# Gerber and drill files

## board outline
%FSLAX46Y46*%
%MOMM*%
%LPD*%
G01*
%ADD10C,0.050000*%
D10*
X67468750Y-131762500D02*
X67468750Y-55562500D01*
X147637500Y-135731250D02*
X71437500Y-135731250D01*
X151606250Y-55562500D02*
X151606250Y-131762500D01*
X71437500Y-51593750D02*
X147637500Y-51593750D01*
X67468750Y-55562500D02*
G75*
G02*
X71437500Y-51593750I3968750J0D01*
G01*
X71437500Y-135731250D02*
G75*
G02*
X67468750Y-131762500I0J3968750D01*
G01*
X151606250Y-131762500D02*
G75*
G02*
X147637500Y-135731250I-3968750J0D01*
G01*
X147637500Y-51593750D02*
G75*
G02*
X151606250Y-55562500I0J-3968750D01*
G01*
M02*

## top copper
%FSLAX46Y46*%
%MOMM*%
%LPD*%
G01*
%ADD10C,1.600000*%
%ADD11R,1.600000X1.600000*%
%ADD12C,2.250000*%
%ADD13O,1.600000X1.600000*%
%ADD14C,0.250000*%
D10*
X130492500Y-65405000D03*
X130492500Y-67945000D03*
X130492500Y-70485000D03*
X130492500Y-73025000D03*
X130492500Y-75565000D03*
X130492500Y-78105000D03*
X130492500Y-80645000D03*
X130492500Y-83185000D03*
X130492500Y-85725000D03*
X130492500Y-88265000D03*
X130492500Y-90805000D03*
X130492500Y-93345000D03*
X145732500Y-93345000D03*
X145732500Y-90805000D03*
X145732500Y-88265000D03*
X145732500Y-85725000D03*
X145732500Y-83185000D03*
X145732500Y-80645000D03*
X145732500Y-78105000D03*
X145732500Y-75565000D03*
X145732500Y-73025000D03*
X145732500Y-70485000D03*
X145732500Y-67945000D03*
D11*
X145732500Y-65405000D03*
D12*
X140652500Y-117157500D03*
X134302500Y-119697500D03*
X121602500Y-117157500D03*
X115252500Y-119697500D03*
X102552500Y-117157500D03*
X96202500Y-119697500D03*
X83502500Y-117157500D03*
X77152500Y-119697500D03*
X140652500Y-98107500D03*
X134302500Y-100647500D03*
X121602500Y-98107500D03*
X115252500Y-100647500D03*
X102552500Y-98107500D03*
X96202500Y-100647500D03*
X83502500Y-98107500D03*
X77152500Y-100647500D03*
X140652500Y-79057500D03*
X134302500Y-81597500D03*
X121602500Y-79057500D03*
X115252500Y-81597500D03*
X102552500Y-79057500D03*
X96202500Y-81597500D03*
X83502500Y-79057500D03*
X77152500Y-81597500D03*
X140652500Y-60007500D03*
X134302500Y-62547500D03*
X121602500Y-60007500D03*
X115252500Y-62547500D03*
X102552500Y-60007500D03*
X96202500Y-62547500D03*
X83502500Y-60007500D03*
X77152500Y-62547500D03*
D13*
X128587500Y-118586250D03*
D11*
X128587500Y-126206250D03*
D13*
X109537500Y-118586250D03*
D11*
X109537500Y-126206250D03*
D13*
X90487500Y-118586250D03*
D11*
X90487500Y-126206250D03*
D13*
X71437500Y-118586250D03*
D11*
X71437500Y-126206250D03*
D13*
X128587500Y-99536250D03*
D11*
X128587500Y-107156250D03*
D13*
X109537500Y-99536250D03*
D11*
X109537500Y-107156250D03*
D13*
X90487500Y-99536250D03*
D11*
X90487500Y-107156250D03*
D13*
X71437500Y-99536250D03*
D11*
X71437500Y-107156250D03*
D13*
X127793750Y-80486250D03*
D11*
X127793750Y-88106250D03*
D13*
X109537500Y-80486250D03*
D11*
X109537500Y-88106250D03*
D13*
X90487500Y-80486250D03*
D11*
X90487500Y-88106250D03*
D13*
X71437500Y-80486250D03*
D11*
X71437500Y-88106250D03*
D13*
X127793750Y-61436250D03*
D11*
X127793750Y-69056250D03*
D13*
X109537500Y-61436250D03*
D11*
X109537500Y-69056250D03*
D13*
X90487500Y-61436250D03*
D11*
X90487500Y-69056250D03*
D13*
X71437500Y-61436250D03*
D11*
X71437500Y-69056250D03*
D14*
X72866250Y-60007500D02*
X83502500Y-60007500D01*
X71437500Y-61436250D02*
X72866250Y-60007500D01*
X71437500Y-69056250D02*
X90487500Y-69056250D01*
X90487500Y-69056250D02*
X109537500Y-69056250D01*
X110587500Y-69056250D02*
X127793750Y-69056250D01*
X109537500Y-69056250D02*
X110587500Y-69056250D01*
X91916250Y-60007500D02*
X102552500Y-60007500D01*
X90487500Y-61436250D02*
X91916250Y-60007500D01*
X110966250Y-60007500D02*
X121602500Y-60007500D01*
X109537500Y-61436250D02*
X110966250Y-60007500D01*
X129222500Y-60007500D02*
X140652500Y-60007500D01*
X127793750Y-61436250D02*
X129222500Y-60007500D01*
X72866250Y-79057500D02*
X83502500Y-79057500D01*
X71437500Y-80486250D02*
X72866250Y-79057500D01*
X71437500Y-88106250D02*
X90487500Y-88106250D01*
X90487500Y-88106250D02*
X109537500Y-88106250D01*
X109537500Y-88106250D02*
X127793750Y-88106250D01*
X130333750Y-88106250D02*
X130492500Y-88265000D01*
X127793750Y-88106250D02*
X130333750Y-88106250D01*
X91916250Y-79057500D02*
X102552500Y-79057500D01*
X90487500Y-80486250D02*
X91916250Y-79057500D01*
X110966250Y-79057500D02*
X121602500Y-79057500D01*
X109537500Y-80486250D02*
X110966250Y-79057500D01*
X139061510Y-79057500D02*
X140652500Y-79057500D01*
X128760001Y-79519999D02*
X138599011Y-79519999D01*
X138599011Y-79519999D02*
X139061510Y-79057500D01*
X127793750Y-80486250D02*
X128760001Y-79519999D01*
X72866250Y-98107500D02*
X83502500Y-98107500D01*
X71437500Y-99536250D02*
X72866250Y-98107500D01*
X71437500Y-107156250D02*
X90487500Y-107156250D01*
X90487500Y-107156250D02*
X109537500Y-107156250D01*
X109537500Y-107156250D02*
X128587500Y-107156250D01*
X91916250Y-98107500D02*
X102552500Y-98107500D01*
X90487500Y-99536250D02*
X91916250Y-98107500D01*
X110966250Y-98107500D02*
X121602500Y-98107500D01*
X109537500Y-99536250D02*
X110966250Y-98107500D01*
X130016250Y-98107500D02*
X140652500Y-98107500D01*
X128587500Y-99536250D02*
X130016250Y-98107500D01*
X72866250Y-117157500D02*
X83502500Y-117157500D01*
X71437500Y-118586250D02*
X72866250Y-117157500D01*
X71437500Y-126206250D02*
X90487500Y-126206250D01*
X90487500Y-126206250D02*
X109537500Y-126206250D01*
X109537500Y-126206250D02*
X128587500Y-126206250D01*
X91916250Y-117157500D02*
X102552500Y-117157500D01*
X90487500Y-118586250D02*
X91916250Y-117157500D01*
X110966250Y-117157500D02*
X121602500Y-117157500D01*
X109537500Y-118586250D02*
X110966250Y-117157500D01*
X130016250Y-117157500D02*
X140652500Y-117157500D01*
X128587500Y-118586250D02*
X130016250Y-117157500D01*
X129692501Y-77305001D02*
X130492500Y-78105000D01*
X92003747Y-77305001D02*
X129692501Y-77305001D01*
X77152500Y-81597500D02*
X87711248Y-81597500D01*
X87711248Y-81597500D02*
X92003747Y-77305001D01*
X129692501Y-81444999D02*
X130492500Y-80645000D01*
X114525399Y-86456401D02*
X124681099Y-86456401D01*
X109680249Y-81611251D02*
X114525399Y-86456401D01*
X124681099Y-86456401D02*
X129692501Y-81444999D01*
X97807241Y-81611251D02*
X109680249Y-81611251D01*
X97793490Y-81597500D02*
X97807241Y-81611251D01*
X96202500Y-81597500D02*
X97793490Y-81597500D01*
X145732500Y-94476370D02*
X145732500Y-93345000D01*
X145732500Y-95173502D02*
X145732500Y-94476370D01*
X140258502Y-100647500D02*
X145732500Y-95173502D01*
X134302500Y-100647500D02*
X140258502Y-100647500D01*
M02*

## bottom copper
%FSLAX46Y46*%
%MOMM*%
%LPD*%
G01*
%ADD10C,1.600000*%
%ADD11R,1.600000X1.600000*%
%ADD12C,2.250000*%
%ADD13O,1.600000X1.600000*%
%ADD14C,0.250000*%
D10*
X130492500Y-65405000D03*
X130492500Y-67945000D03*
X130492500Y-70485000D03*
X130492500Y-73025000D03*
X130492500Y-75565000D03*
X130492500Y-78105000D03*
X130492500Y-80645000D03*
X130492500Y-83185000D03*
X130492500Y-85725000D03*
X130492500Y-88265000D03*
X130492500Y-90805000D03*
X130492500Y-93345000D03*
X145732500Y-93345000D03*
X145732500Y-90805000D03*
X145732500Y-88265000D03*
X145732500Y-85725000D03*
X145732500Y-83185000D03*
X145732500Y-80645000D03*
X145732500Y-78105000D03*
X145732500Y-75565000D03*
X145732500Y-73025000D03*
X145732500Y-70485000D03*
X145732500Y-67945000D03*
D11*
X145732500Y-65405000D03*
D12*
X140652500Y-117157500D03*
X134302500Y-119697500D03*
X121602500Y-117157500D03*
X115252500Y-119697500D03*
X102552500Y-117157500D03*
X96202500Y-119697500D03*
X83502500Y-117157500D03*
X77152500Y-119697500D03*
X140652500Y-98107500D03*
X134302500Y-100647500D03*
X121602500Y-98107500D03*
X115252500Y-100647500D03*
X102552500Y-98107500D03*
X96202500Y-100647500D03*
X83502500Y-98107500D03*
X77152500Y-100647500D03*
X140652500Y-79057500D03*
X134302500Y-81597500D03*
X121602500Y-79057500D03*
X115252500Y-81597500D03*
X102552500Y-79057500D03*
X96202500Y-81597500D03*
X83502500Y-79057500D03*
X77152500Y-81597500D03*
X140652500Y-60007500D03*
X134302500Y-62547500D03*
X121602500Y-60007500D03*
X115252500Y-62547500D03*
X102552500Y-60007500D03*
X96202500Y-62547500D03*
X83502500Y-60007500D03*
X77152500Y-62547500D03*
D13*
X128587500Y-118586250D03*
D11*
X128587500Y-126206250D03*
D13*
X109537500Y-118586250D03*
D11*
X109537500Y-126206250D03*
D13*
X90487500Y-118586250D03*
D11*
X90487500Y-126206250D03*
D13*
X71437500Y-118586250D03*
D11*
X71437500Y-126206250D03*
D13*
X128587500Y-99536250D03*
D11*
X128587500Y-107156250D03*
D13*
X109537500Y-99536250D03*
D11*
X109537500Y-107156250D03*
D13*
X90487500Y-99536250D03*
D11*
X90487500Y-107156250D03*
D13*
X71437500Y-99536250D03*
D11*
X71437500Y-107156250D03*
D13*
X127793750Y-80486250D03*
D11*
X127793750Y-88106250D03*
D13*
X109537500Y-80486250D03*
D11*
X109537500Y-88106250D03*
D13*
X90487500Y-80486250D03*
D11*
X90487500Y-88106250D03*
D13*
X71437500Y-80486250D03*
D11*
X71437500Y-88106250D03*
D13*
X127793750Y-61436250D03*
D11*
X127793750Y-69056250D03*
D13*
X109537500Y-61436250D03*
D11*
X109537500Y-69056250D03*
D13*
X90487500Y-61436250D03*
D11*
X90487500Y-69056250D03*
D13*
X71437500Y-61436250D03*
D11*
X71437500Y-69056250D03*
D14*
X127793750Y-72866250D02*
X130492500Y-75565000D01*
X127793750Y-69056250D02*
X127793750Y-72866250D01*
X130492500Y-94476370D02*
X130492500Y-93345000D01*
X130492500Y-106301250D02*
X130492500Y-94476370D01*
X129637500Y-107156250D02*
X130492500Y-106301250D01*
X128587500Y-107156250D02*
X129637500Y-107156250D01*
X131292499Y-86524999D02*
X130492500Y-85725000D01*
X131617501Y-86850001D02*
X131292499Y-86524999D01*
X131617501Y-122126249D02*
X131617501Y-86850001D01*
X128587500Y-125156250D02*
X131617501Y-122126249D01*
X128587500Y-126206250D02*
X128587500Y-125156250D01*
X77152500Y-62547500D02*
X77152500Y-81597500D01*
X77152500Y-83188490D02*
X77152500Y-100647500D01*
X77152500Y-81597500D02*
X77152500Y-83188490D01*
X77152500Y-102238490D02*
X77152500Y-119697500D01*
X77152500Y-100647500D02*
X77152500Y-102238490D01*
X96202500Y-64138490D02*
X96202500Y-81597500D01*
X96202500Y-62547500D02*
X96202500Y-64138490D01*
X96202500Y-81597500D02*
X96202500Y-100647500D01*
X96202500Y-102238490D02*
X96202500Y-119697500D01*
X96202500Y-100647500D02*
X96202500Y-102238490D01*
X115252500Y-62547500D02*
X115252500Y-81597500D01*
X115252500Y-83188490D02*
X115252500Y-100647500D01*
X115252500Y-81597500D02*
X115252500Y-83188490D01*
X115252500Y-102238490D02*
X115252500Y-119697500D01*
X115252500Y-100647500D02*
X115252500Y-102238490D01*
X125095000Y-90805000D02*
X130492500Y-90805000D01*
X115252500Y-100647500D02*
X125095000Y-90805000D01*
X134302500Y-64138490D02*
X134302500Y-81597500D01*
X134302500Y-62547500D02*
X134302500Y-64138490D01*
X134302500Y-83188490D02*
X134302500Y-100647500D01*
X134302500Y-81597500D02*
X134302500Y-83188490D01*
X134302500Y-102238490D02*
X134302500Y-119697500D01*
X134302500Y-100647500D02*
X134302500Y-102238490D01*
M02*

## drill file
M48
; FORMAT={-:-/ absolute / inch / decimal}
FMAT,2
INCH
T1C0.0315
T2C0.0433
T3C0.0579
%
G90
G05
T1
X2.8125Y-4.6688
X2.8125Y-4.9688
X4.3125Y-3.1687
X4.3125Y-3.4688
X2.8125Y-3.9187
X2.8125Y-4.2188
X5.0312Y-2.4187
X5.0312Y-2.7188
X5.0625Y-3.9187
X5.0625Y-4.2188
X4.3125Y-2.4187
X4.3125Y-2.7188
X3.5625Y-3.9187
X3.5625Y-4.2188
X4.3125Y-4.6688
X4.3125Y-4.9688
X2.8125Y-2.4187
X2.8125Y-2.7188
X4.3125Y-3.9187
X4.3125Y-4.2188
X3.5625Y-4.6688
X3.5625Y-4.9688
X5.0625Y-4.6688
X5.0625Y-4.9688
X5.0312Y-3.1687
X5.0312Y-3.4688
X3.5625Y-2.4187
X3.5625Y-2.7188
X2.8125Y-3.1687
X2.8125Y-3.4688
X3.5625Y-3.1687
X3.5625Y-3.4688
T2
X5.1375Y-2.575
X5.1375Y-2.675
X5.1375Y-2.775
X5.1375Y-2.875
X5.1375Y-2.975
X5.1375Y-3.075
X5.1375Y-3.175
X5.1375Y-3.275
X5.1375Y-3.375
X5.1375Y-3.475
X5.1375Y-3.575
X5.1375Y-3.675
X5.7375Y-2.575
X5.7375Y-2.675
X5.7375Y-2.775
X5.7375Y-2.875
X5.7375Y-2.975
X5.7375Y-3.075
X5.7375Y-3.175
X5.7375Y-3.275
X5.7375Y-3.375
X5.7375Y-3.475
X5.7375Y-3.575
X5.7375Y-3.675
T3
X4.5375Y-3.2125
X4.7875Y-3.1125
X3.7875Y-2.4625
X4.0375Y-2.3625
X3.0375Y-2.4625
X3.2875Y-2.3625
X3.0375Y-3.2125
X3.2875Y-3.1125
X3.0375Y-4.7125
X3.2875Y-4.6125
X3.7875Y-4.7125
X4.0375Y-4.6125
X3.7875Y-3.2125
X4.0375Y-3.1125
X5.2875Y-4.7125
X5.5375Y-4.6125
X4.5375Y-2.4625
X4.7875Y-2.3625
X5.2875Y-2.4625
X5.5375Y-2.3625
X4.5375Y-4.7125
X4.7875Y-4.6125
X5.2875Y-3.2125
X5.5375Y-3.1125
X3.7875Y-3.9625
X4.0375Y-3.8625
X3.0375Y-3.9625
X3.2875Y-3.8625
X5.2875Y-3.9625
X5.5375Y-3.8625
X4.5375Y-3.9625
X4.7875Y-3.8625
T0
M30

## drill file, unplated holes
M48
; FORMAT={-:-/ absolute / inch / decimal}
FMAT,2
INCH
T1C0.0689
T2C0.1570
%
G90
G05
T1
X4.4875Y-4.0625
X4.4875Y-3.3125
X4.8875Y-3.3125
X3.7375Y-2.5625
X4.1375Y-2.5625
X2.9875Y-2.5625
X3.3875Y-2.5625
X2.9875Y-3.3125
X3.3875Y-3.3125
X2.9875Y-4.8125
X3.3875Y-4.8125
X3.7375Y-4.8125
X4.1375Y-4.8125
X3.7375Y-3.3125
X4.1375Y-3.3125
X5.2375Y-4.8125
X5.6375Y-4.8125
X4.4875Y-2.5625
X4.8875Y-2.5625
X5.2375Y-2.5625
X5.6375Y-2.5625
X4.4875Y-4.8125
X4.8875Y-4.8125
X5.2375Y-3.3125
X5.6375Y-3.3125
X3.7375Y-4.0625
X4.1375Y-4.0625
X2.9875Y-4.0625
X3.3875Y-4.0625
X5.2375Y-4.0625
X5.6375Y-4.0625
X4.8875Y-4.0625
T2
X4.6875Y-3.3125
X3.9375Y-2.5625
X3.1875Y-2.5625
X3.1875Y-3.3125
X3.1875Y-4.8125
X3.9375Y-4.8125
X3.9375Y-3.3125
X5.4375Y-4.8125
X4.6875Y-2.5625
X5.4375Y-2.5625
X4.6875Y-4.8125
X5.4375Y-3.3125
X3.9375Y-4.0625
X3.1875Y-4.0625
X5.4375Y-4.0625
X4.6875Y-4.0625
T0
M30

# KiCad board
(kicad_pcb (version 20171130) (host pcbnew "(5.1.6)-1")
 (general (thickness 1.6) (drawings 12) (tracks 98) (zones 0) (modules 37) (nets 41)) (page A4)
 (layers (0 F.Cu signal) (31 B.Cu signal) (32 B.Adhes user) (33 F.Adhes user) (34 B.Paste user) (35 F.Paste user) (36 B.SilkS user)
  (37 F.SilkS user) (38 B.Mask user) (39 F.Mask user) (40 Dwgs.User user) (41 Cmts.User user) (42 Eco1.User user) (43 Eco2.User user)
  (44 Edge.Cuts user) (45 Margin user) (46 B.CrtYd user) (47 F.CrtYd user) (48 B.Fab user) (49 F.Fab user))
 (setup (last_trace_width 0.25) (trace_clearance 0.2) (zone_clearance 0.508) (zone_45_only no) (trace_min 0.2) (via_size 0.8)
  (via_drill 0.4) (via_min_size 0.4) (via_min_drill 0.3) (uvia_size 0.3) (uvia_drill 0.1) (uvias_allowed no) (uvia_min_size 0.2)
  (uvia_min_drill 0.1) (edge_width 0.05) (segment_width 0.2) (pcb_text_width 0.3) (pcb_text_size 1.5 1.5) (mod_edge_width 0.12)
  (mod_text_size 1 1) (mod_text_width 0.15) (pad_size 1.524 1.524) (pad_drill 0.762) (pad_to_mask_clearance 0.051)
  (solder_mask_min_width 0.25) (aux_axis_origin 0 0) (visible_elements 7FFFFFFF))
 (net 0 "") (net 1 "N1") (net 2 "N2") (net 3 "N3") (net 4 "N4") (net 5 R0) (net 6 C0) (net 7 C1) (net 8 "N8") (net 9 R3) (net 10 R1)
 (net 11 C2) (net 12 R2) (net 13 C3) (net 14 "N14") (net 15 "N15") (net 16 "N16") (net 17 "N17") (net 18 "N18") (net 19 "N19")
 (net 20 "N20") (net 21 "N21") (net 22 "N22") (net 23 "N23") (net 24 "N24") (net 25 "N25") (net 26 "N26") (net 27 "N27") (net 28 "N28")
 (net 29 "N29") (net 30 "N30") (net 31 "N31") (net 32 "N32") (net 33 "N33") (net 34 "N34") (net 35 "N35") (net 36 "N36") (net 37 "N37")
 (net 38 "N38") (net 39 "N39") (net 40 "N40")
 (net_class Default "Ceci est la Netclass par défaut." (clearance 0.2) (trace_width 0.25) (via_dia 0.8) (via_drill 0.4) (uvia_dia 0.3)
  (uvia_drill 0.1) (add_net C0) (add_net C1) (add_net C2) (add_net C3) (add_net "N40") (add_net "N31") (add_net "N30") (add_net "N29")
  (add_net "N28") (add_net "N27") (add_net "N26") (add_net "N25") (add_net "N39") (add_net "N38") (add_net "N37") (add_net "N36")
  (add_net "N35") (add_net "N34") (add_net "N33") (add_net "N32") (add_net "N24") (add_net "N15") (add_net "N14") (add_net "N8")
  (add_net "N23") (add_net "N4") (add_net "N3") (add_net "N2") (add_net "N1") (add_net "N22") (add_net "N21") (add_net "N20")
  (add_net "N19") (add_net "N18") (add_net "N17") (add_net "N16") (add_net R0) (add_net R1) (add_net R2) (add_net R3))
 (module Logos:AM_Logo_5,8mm (layer B.Cu) (at 109.5375 130.96875 180)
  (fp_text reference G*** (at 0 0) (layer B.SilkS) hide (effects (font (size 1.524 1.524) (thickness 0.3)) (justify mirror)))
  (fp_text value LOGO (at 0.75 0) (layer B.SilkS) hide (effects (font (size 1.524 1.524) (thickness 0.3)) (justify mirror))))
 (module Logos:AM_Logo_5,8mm (layer F.Cu) (at 109.5375 130.96875)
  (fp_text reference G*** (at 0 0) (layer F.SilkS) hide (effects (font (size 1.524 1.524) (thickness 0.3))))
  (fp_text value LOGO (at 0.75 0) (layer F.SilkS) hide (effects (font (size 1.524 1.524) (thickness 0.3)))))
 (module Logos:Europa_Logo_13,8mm (layer B.Cu) (at 109.5375 93.6625 180)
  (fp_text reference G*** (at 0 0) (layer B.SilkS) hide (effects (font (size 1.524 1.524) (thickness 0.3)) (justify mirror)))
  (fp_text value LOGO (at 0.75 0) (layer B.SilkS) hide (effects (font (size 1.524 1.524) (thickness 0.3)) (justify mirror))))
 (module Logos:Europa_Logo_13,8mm (layer F.Cu) (at 109.5375 93.6625)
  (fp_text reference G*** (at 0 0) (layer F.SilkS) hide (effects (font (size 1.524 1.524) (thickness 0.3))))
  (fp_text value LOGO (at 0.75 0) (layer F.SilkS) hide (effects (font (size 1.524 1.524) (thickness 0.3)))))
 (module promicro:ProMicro (layer B.Cu) (at 138.1125 79.375 270)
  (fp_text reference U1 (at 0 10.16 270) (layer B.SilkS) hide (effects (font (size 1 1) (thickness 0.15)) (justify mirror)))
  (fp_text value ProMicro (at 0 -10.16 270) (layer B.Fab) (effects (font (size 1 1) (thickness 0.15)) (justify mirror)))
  (pad 24 thru_hole circle (at -13.97 7.62 270) (size 1.6 1.6) (drill 1.1) (layers *.Cu *.Mask B.SilkS) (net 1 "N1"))
  (pad 23 thru_hole circle (at -11.43 7.62 270) (size 1.6 1.6) (drill 1.1) (layers *.Cu *.Mask B.SilkS) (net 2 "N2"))
  (pad 22 thru_hole circle (at -8.89 7.62 270) (size 1.6 1.6) (drill 1.1) (layers *.Cu *.Mask B.SilkS) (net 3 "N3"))
  (pad 21 thru_hole circle (at -6.35 7.62 270) (size 1.6 1.6) (drill 1.1) (layers *.Cu *.Mask B.SilkS) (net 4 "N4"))
  (pad 20 thru_hole circle (at -3.81 7.62 270) (size 1.6 1.6) (drill 1.1) (layers *.Cu *.Mask B.SilkS) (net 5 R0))
  (pad 19 thru_hole circle (at -1.27 7.62 270) (size 1.6 1.6) (drill 1.1) (layers *.Cu *.Mask B.SilkS) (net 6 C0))
  (pad 18 thru_hole circle (at 1.27 7.62 270) (size 1.6 1.6) (drill 1.1) (layers *.Cu *.Mask B.SilkS) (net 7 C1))
  (pad 17 thru_hole circle (at 3.81 7.62 270) (size 1.6 1.6) (drill 1.1) (layers *.Cu *.Mask B.SilkS) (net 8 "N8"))
  (pad 16 thru_hole circle (at 6.35 7.62 270) (size 1.6 1.6) (drill 1.1) (layers *.Cu *.Mask B.SilkS) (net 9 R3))
  (pad 15 thru_hole circle (at 8.89 7.62 270) (size 1.6 1.6) (drill 1.1) (layers *.Cu *.Mask B.SilkS) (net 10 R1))
  (pad 14 thru_hole circle (at 11.43 7.62 270) (size 1.6 1.6) (drill 1.1) (layers *.Cu *.Mask B.SilkS) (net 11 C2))
  (pad 13 thru_hole circle (at 13.97 7.62 270) (size 1.6 1.6) (drill 1.1) (layers *.Cu *.Mask B.SilkS) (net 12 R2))
  (pad 12 thru_hole circle (at 13.97 -7.62 270) (size 1.6 1.6) (drill 1.1) (layers *.Cu *.Mask B.SilkS) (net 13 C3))
  (pad 11 thru_hole circle (at 11.43 -7.62 270) (size 1.6 1.6) (drill 1.1) (layers *.Cu *.Mask B.SilkS) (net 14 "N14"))
  (pad 10 thru_hole circle (at 8.89 -7.62 270) (size 1.6 1.6) (drill 1.1) (layers *.Cu *.Mask B.SilkS) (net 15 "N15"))
  (pad 9 thru_hole circle (at 6.35 -7.62 270) (size 1.6 1.6) (drill 1.1) (layers *.Cu *.Mask B.SilkS) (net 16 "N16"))
  (pad 8 thru_hole circle (at 3.81 -7.62 270) (size 1.6 1.6) (drill 1.1) (layers *.Cu *.Mask B.SilkS) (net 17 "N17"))
  (pad 7 thru_hole circle (at 1.27 -7.62 270) (size 1.6 1.6) (drill 1.1) (layers *.Cu *.Mask B.SilkS) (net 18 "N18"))
  (pad 6 thru_hole circle (at -1.27 -7.62 270) (size 1.6 1.6) (drill 1.1) (layers *.Cu *.Mask B.SilkS) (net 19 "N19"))
  (pad 5 thru_hole circle (at -3.81 -7.62 270) (size 1.6 1.6) (drill 1.1) (layers *.Cu *.Mask B.SilkS) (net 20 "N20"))
  (pad 4 thru_hole circle (at -6.35 -7.62 270) (size 1.6 1.6) (drill 1.1) (layers *.Cu *.Mask B.SilkS) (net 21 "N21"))
  (pad 3 thru_hole circle (at -8.89 -7.62 270) (size 1.6 1.6) (drill 1.1) (layers *.Cu *.Mask B.SilkS) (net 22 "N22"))
  (pad 2 thru_hole circle (at -11.43 -7.62 270) (size 1.6 1.6) (drill 1.1) (layers *.Cu *.Mask B.SilkS) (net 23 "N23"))
  (pad 1 thru_hole rect (at -13.97 -7.62 270) (size 1.6 1.6) (drill 1.1) (layers *.Cu *.Mask B.SilkS) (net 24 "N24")))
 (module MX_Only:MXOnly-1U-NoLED (layer F.Cu) (at 138.1125 122.2375)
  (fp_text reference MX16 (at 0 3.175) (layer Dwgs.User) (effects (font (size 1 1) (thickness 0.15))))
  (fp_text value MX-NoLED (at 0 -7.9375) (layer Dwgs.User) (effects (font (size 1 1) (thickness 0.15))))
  (pad 2 thru_hole circle (at 2.54 -5.08) (size 2.25 2.25) (drill 1.47) (layers *.Cu B.Mask) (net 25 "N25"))
  (pad "" np_thru_hole circle (at 0 0) (size 3.9878 3.9878) (drill 3.9878) (layers *.Cu *.Mask))
  (pad 1 thru_hole circle (at -3.81 -2.54) (size 2.25 2.25) (drill 1.47) (layers *.Cu B.Mask) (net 13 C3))
  (pad "" np_thru_hole circle (at -5.08 0 48.0996) (size 1.75 1.75) (drill 1.75) (layers *.Cu *.Mask))
  (pad "" np_thru_hole circle (at 5.08 0 48.0996) (size 1.75 1.75) (drill 1.75) (layers *.Cu *.Mask)))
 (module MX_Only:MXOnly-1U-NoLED (layer F.Cu) (at 119.0625 122.2375)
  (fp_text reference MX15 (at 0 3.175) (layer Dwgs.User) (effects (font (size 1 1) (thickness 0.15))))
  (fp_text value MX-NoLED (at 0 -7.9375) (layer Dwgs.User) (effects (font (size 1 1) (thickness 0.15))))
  (pad 2 thru_hole circle (at 2.54 -5.08) (size 2.25 2.25) (drill 1.47) (layers *.Cu B.Mask) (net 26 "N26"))
  (pad "" np_thru_hole circle (at 0 0) (size 3.9878 3.9878) (drill 3.9878) (layers *.Cu *.Mask))
  (pad 1 thru_hole circle (at -3.81 -2.54) (size 2.25 2.25) (drill 1.47) (layers *.Cu B.Mask) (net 11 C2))
  (pad "" np_thru_hole circle (at -5.08 0 48.0996) (size 1.75 1.75) (drill 1.75) (layers *.Cu *.Mask))
  (pad "" np_thru_hole circle (at 5.08 0 48.0996) (size 1.75 1.75) (drill 1.75) (layers *.Cu *.Mask)))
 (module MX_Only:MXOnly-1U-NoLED (layer F.Cu) (at 100.0125 122.2375)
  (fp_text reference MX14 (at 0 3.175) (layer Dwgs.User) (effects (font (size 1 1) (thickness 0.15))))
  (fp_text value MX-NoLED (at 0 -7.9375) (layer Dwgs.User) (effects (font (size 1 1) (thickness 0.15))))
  (pad 2 thru_hole circle (at 2.54 -5.08) (size 2.25 2.25) (drill 1.47) (layers *.Cu B.Mask) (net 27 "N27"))
  (pad "" np_thru_hole circle (at 0 0) (size 3.9878 3.9878) (drill 3.9878) (layers *.Cu *.Mask))
  (pad 1 thru_hole circle (at -3.81 -2.54) (size 2.25 2.25) (drill 1.47) (layers *.Cu B.Mask) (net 7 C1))
  (pad "" np_thru_hole circle (at -5.08 0 48.0996) (size 1.75 1.75) (drill 1.75) (layers *.Cu *.Mask))
  (pad "" np_thru_hole circle (at 5.08 0 48.0996) (size 1.75 1.75) (drill 1.75) (layers *.Cu *.Mask)))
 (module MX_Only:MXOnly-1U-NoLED (layer F.Cu) (at 80.9625 122.2375)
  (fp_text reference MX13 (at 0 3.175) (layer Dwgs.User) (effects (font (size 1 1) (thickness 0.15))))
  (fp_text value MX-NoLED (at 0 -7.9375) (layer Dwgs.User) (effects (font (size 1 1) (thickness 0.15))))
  (pad 2 thru_hole circle (at 2.54 -5.08) (size 2.25 2.25) (drill 1.47) (layers *.Cu B.Mask) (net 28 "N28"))
  (pad "" np_thru_hole circle (at 0 0) (size 3.9878 3.9878) (drill 3.9878) (layers *.Cu *.Mask))
  (pad 1 thru_hole circle (at -3.81 -2.54) (size 2.25 2.25) (drill 1.47) (layers *.Cu B.Mask) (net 6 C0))
  (pad "" np_thru_hole circle (at -5.08 0 48.0996) (size 1.75 1.75) (drill 1.75) (layers *.Cu *.Mask))
  (pad "" np_thru_hole circle (at 5.08 0 48.0996) (size 1.75 1.75) (drill 1.75) (layers *.Cu *.Mask)))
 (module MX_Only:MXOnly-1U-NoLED (layer F.Cu) (at 138.1125 103.1875)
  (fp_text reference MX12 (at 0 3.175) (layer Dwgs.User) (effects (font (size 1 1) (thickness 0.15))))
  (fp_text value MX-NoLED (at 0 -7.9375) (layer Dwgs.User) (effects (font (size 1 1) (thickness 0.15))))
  (pad 2 thru_hole circle (at 2.54 -5.08) (size 2.25 2.25) (drill 1.47) (layers *.Cu B.Mask) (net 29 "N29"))
  (pad "" np_thru_hole circle (at 0 0) (size 3.9878 3.9878) (drill 3.9878) (layers *.Cu *.Mask))
  (pad 1 thru_hole circle (at -3.81 -2.54) (size 2.25 2.25) (drill 1.47) (layers *.Cu B.Mask) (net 13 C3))
  (pad "" np_thru_hole circle (at -5.08 0 48.0996) (size 1.75 1.75) (drill 1.75) (layers *.Cu *.Mask))
  (pad "" np_thru_hole circle (at 5.08 0 48.0996) (size 1.75 1.75) (drill 1.75) (layers *.Cu *.Mask)))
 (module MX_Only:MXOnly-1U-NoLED (layer F.Cu) (at 119.0625 103.1875)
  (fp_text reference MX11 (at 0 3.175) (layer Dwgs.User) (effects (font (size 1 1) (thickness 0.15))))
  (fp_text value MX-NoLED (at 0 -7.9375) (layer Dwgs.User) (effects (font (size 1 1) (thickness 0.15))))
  (pad 2 thru_hole circle (at 2.54 -5.08) (size 2.25 2.25) (drill 1.47) (layers *.Cu B.Mask) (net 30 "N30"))
  (pad "" np_thru_hole circle (at 0 0) (size 3.9878 3.9878) (drill 3.9878) (layers *.Cu *.Mask))
  (pad 1 thru_hole circle (at -3.81 -2.54) (size 2.25 2.25) (drill 1.47) (layers *.Cu B.Mask) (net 11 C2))
  (pad "" np_thru_hole circle (at -5.08 0 48.0996) (size 1.75 1.75) (drill 1.75) (layers *.Cu *.Mask))
  (pad "" np_thru_hole circle (at 5.08 0 48.0996) (size 1.75 1.75) (drill 1.75) (layers *.Cu *.Mask)))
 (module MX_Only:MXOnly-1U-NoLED (layer F.Cu) (at 100.0125 103.1875)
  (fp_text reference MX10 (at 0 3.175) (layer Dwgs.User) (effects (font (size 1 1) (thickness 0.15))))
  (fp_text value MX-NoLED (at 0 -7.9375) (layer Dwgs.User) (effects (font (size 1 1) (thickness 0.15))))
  (pad 2 thru_hole circle (at 2.54 -5.08) (size 2.25 2.25) (drill 1.47) (layers *.Cu B.Mask) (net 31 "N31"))
  (pad "" np_thru_hole circle (at 0 0) (size 3.9878 3.9878) (drill 3.9878) (layers *.Cu *.Mask))
  (pad 1 thru_hole circle (at -3.81 -2.54) (size 2.25 2.25) (drill 1.47) (layers *.Cu B.Mask) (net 7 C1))
  (pad "" np_thru_hole circle (at -5.08 0 48.0996) (size 1.75 1.75) (drill 1.75) (layers *.Cu *.Mask))
  (pad "" np_thru_hole circle (at 5.08 0 48.0996) (size 1.75 1.75) (drill 1.75) (layers *.Cu *.Mask)))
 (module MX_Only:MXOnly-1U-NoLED (layer F.Cu) (at 80.9625 103.1875)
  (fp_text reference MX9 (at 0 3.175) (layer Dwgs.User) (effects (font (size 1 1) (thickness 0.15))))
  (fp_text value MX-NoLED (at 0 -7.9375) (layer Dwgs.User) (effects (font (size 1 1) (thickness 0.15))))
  (pad 2 thru_hole circle (at 2.54 -5.08) (size 2.25 2.25) (drill 1.47) (layers *.Cu B.Mask) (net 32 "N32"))
  (pad "" np_thru_hole circle (at 0 0) (size 3.9878 3.9878) (drill 3.9878) (layers *.Cu *.Mask))
  (pad 1 thru_hole circle (at -3.81 -2.54) (size 2.25 2.25) (drill 1.47) (layers *.Cu B.Mask) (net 6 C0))
  (pad "" np_thru_hole circle (at -5.08 0 48.0996) (size 1.75 1.75) (drill 1.75) (layers *.Cu *.Mask))
  (pad "" np_thru_hole circle (at 5.08 0 48.0996) (size 1.75 1.75) (drill 1.75) (layers *.Cu *.Mask)))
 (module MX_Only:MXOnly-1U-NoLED (layer F.Cu) (at 138.1125 84.1375)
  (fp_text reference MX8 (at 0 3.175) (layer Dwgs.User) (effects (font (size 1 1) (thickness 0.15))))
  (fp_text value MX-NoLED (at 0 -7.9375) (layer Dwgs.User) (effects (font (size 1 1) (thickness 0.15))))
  (pad 2 thru_hole circle (at 2.54 -5.08) (size 2.25 2.25) (drill 1.47) (layers *.Cu B.Mask) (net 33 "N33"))
  (pad "" np_thru_hole circle (at 0 0) (size 3.9878 3.9878) (drill 3.9878) (layers *.Cu *.Mask))
  (pad 1 thru_hole circle (at -3.81 -2.54) (size 2.25 2.25) (drill 1.47) (layers *.Cu B.Mask) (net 13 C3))
  (pad "" np_thru_hole circle (at -5.08 0 48.0996) (size 1.75 1.75) (drill 1.75) (layers *.Cu *.Mask))
  (pad "" np_thru_hole circle (at 5.08 0 48.0996) (size 1.75 1.75) (drill 1.75) (layers *.Cu *.Mask)))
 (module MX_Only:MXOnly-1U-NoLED (layer F.Cu) (at 119.0625 84.1375)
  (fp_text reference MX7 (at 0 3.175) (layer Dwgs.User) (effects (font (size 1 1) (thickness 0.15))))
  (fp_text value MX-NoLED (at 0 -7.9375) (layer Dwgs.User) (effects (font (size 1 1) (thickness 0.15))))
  (pad 2 thru_hole circle (at 2.54 -5.08) (size 2.25 2.25) (drill 1.47) (layers *.Cu B.Mask) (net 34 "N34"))
  (pad "" np_thru_hole circle (at 0 0) (size 3.9878 3.9878) (drill 3.9878) (layers *.Cu *.Mask))
  (pad 1 thru_hole circle (at -3.81 -2.54) (size 2.25 2.25) (drill 1.47) (layers *.Cu B.Mask) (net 11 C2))
  (pad "" np_thru_hole circle (at -5.08 0 48.0996) (size 1.75 1.75) (drill 1.75) (layers *.Cu *.Mask))
  (pad "" np_thru_hole circle (at 5.08 0 48.0996) (size 1.75 1.75) (drill 1.75) (layers *.Cu *.Mask)))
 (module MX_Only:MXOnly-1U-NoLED (layer F.Cu) (at 100.0125 84.1375)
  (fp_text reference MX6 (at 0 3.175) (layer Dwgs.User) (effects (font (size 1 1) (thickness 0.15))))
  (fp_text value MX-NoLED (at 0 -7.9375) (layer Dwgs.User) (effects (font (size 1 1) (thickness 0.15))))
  (pad 2 thru_hole circle (at 2.54 -5.08) (size 2.25 2.25) (drill 1.47) (layers *.Cu B.Mask) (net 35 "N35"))
  (pad "" np_thru_hole circle (at 0 0) (size 3.9878 3.9878) (drill 3.9878) (layers *.Cu *.Mask))
  (pad 1 thru_hole circle (at -3.81 -2.54) (size 2.25 2.25) (drill 1.47) (layers *.Cu B.Mask) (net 7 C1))
  (pad "" np_thru_hole circle (at -5.08 0 48.0996) (size 1.75 1.75) (drill 1.75) (layers *.Cu *.Mask))
  (pad "" np_thru_hole circle (at 5.08 0 48.0996) (size 1.75 1.75) (drill 1.75) (layers *.Cu *.Mask)))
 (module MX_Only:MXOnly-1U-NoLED (layer F.Cu) (at 80.9625 84.1375)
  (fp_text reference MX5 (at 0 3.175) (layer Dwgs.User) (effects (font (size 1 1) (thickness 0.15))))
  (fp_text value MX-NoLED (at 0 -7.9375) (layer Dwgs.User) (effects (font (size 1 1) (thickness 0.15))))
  (pad 2 thru_hole circle (at 2.54 -5.08) (size 2.25 2.25) (drill 1.47) (layers *.Cu B.Mask) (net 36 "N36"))
  (pad "" np_thru_hole circle (at 0 0) (size 3.9878 3.9878) (drill 3.9878) (layers *.Cu *.Mask))
  (pad 1 thru_hole circle (at -3.81 -2.54) (size 2.25 2.25) (drill 1.47) (layers *.Cu B.Mask) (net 6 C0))
  (pad "" np_thru_hole circle (at -5.08 0 48.0996) (size 1.75 1.75) (drill 1.75) (layers *.Cu *.Mask))
  (pad "" np_thru_hole circle (at 5.08 0 48.0996) (size 1.75 1.75) (drill 1.75) (layers *.Cu *.Mask)))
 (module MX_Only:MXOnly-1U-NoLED (layer F.Cu) (at 138.1125 65.0875)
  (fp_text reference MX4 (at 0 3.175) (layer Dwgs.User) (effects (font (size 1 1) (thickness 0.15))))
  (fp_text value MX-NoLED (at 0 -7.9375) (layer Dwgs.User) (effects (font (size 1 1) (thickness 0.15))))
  (pad 2 thru_hole circle (at 2.54 -5.08) (size 2.25 2.25) (drill 1.47) (layers *.Cu B.Mask) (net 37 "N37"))
  (pad "" np_thru_hole circle (at 0 0) (size 3.9878 3.9878) (drill 3.9878) (layers *.Cu *.Mask))
  (pad 1 thru_hole circle (at -3.81 -2.54) (size 2.25 2.25) (drill 1.47) (layers *.Cu B.Mask) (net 13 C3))
  (pad "" np_thru_hole circle (at -5.08 0 48.0996) (size 1.75 1.75) (drill 1.75) (layers *.Cu *.Mask))
  (pad "" np_thru_hole circle (at 5.08 0 48.0996) (size 1.75 1.75) (drill 1.75) (layers *.Cu *.Mask)))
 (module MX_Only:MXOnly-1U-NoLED (layer F.Cu) (at 119.0625 65.0875)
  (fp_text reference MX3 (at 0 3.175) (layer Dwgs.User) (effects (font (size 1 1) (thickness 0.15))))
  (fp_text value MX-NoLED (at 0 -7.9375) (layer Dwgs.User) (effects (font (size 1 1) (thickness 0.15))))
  (pad 2 thru_hole circle (at 2.54 -5.08) (size 2.25 2.25) (drill 1.47) (layers *.Cu B.Mask) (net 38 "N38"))
  (pad "" np_thru_hole circle (at 0 0) (size 3.9878 3.9878) (drill 3.9878) (layers *.Cu *.Mask))
  (pad 1 thru_hole circle (at -3.81 -2.54) (size 2.25 2.25) (drill 1.47) (layers *.Cu B.Mask) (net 11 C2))
  (pad "" np_thru_hole circle (at -5.08 0 48.0996) (size 1.75 1.75) (drill 1.75) (layers *.Cu *.Mask))
  (pad "" np_thru_hole circle (at 5.08 0 48.0996) (size 1.75 1.75) (drill 1.75) (layers *.Cu *.Mask)))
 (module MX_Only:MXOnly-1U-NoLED (layer F.Cu) (at 100.0125 65.0875)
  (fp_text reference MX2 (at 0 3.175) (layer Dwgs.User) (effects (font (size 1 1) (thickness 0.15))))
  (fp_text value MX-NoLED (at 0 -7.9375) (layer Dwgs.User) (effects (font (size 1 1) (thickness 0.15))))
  (pad 2 thru_hole circle (at 2.54 -5.08) (size 2.25 2.25) (drill 1.47) (layers *.Cu B.Mask) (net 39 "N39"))
  (pad "" np_thru_hole circle (at 0 0) (size 3.9878 3.9878) (drill 3.9878) (layers *.Cu *.Mask))
  (pad 1 thru_hole circle (at -3.81 -2.54) (size 2.25 2.25) (drill 1.47) (layers *.Cu B.Mask) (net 7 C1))
  (pad "" np_thru_hole circle (at -5.08 0 48.0996) (size 1.75 1.75) (drill 1.75) (layers *.Cu *.Mask))
  (pad "" np_thru_hole circle (at 5.08 0 48.0996) (size 1.75 1.75) (drill 1.75) (layers *.Cu *.Mask)))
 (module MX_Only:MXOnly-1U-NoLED (layer F.Cu) (at 80.9625 65.0875)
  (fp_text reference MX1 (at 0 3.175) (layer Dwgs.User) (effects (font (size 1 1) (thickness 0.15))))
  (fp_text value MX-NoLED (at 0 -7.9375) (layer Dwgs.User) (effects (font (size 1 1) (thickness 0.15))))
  (pad 2 thru_hole circle (at 2.54 -5.08) (size 2.25 2.25) (drill 1.47) (layers *.Cu B.Mask) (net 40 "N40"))
  (pad "" np_thru_hole circle (at 0 0) (size 3.9878 3.9878) (drill 3.9878) (layers *.Cu *.Mask))
  (pad 1 thru_hole circle (at -3.81 -2.54) (size 2.25 2.25) (drill 1.47) (layers *.Cu B.Mask) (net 6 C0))
  (pad "" np_thru_hole circle (at -5.08 0 48.0996) (size 1.75 1.75) (drill 1.75) (layers *.Cu *.Mask))
  (pad "" np_thru_hole circle (at 5.08 0 48.0996) (size 1.75 1.75) (drill 1.75) (layers *.Cu *.Mask)))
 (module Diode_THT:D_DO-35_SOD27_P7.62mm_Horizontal (layer B.Cu) (at 128.5875 126.20625 90)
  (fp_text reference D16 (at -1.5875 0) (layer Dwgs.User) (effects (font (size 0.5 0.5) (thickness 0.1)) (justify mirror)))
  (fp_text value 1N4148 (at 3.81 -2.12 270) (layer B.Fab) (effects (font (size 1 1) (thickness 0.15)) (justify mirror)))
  (pad 2 thru_hole oval (at 7.62 0 90) (size 1.6 1.6) (drill 0.8) (layers *.Cu *.Mask) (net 25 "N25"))
  (pad 1 thru_hole rect (at 0 0 90) (size 1.6 1.6) (drill 0.8) (layers *.Cu *.Mask) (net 9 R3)))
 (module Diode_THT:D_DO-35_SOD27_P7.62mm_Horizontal (layer B.Cu) (at 109.5375 126.20625 90)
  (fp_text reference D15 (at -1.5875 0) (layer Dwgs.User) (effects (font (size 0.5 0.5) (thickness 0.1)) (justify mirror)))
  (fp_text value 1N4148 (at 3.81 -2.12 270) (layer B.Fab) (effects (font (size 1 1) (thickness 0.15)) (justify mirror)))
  (pad 2 thru_hole oval (at 7.62 0 90) (size 1.6 1.6) (drill 0.8) (layers *.Cu *.Mask) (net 26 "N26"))
  (pad 1 thru_hole rect (at 0 0 90) (size 1.6 1.6) (drill 0.8) (layers *.Cu *.Mask) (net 9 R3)))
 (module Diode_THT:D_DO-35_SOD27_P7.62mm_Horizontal (layer B.Cu) (at 90.4875 126.20625 90)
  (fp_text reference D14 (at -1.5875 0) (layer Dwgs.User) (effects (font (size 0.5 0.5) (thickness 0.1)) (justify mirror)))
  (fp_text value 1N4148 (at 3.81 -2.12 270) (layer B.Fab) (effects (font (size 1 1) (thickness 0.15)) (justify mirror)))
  (pad 2 thru_hole oval (at 7.62 0 90) (size 1.6 1.6) (drill 0.8) (layers *.Cu *.Mask) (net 27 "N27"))
  (pad 1 thru_hole rect (at 0 0 90) (size 1.6 1.6) (drill 0.8) (layers *.Cu *.Mask) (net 9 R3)))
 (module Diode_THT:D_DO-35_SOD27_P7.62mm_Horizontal (layer B.Cu) (at 71.4375 126.20625 90)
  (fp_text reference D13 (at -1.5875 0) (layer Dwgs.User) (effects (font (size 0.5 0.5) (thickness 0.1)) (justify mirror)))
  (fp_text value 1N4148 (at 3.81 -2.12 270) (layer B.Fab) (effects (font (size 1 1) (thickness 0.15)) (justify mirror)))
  (pad 2 thru_hole oval (at 7.62 0 90) (size 1.6 1.6) (drill 0.8) (layers *.Cu *.Mask) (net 28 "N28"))
  (pad 1 thru_hole rect (at 0 0 90) (size 1.6 1.6) (drill 0.8) (layers *.Cu *.Mask) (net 9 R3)))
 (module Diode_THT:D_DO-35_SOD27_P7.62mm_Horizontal (layer B.Cu) (at 128.5875 107.15625 90)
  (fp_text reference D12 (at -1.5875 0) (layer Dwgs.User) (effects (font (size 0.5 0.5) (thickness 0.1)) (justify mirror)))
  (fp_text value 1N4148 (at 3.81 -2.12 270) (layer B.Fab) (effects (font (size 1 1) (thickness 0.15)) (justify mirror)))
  (pad 2 thru_hole oval (at 7.62 0 90) (size 1.6 1.6) (drill 0.8) (layers *.Cu *.Mask) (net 29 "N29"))
  (pad 1 thru_hole rect (at 0 0 90) (size 1.6 1.6) (drill 0.8) (layers *.Cu *.Mask) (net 12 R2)))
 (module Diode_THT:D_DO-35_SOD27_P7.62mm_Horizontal (layer B.Cu) (at 109.5375 107.15625 90)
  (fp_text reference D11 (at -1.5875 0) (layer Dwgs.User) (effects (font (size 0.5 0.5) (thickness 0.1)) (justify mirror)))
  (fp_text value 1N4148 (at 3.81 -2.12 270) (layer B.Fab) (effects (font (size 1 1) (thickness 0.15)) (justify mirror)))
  (pad 2 thru_hole oval (at 7.62 0 90) (size 1.6 1.6) (drill 0.8) (layers *.Cu *.Mask) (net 30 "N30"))
  (pad 1 thru_hole rect (at 0 0 90) (size 1.6 1.6) (drill 0.8) (layers *.Cu *.Mask) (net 12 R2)))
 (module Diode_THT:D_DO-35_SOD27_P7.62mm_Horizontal (layer B.Cu) (at 90.4875 107.15625 90)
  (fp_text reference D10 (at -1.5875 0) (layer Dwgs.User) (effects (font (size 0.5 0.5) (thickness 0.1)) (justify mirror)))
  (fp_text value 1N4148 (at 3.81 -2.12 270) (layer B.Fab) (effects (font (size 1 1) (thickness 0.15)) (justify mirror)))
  (pad 2 thru_hole oval (at 7.62 0 90) (size 1.6 1.6) (drill 0.8) (layers *.Cu *.Mask) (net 31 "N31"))
  (pad 1 thru_hole rect (at 0 0 90) (size 1.6 1.6) (drill 0.8) (layers *.Cu *.Mask) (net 12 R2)))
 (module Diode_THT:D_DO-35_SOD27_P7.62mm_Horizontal (layer B.Cu) (at 71.4375 107.15625 90)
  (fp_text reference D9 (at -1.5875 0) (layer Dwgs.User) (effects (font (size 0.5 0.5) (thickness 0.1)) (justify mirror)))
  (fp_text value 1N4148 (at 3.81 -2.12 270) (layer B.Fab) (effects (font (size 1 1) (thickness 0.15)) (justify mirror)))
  (pad 2 thru_hole oval (at 7.62 0 90) (size 1.6 1.6) (drill 0.8) (layers *.Cu *.Mask) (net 32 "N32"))
  (pad 1 thru_hole rect (at 0 0 90) (size 1.6 1.6) (drill 0.8) (layers *.Cu *.Mask) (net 12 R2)))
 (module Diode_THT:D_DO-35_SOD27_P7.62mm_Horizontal (layer B.Cu) (at 127.79375 88.10625 90)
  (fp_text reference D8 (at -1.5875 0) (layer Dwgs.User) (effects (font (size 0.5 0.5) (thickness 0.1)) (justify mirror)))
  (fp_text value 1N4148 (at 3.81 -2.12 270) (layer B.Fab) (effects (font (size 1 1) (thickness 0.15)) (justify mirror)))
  (pad 2 thru_hole oval (at 7.62 0 90) (size 1.6 1.6) (drill 0.8) (layers *.Cu *.Mask) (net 33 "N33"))
  (pad 1 thru_hole rect (at 0 0 90) (size 1.6 1.6) (drill 0.8) (layers *.Cu *.Mask) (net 10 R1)))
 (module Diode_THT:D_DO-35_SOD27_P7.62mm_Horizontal (layer B.Cu) (at 109.5375 88.10625 90)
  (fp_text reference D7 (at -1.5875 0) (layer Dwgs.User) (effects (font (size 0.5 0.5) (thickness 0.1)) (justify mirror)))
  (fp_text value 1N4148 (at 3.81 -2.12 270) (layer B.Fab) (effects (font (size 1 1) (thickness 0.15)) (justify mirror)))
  (pad 2 thru_hole oval (at 7.62 0 90) (size 1.6 1.6) (drill 0.8) (layers *.Cu *.Mask) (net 34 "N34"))
  (pad 1 thru_hole rect (at 0 0 90) (size 1.6 1.6) (drill 0.8) (layers *.Cu *.Mask) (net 10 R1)))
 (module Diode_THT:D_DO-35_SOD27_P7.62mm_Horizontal (layer B.Cu) (at 90.4875 88.10625 90)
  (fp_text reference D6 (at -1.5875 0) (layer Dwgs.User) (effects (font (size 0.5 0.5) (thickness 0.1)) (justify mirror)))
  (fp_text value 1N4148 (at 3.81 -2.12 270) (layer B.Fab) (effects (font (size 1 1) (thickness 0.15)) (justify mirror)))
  (pad 2 thru_hole oval (at 7.62 0 90) (size 1.6 1.6) (drill 0.8) (layers *.Cu *.Mask) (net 35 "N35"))
  (pad 1 thru_hole rect (at 0 0 90) (size 1.6 1.6) (drill 0.8) (layers *.Cu *.Mask) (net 10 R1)))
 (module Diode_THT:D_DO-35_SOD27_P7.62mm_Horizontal (layer B.Cu) (at 71.4375 88.10625 90)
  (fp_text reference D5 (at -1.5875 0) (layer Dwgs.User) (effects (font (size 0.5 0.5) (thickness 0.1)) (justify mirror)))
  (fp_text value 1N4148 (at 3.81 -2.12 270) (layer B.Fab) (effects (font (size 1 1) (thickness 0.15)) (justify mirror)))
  (pad 2 thru_hole oval (at 7.62 0 90) (size 1.6 1.6) (drill 0.8) (layers *.Cu *.Mask) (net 36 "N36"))
  (pad 1 thru_hole rect (at 0 0 90) (size 1.6 1.6) (drill 0.8) (layers *.Cu *.Mask) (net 10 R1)))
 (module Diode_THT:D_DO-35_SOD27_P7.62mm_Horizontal (layer B.Cu) (at 127.79375 69.05625 90)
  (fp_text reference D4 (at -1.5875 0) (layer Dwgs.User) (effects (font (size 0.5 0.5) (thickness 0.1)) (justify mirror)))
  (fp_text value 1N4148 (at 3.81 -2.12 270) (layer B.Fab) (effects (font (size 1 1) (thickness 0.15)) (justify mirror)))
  (pad 2 thru_hole oval (at 7.62 0 90) (size 1.6 1.6) (drill 0.8) (layers *.Cu *.Mask) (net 37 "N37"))
  (pad 1 thru_hole rect (at 0 0 90) (size 1.6 1.6) (drill 0.8) (layers *.Cu *.Mask) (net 5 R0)))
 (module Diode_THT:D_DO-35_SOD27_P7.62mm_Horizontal (layer B.Cu) (at 109.5375 69.05625 90)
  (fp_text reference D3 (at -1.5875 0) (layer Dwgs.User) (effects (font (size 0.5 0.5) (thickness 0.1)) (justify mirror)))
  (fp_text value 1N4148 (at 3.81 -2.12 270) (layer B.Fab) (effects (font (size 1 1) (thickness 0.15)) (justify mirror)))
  (pad 2 thru_hole oval (at 7.62 0 90) (size 1.6 1.6) (drill 0.8) (layers *.Cu *.Mask) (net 38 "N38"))
  (pad 1 thru_hole rect (at 0 0 90) (size 1.6 1.6) (drill 0.8) (layers *.Cu *.Mask) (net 5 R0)))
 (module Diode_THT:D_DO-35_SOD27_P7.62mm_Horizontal (layer B.Cu) (at 90.4875 69.05625 90)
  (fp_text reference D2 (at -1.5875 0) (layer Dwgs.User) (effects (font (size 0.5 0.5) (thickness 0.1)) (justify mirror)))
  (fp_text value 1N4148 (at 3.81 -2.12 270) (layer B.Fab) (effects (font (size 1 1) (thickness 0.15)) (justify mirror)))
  (pad 2 thru_hole oval (at 7.62 0 90) (size 1.6 1.6) (drill 0.8) (layers *.Cu *.Mask) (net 39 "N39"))
  (pad 1 thru_hole rect (at 0 0 90) (size 1.6 1.6) (drill 0.8) (layers *.Cu *.Mask) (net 5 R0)))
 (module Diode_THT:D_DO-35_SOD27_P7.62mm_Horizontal (layer B.Cu) (at 71.4375 69.05625 90)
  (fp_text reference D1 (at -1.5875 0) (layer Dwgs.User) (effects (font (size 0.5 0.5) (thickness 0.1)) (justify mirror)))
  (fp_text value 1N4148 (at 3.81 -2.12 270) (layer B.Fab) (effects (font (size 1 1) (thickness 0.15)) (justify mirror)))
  (pad 2 thru_hole oval (at 7.62 0 90) (size 1.6 1.6) (drill 0.8) (layers *.Cu *.Mask) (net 40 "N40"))
  (pad 1 thru_hole rect (at 0 0 90) (size 1.6 1.6) (drill 0.8) (layers *.Cu *.Mask) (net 5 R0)))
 (gr_line (start 67.46875 131.7625) (end 67.46875 55.5625) (layer Edge.Cuts) (width 0.05))
 (gr_line (start 147.6375 135.73125) (end 71.4375 135.73125) (layer Edge.Cuts) (width 0.05))
 (gr_line (start 151.60625 55.5625) (end 151.60625 131.7625) (layer Edge.Cuts) (width 0.05))
 (gr_line (start 71.4375 51.59375) (end 147.6375 51.59375) (layer Edge.Cuts) (width 0.05))
 (gr_arc (start 71.4375 55.5625) (end 71.4375 51.59375) (angle -90) (layer Edge.Cuts) (width 0.05))
 (gr_arc (start 71.4375 131.7625) (end 67.46875 131.7625) (angle -90) (layer Edge.Cuts) (width 0.05))
 (gr_arc (start 147.6375 131.7625) (end 147.6375 135.73125) (angle -90) (layer Edge.Cuts) (width 0.05))
 (gr_arc (start 147.6375 55.5625) (end 151.60625 55.5625) (angle -90) (layer Edge.Cuts) (width 0.05))
 (segment (start 72.86625 60.0075) (end 83.5025 60.0075) (width 0.25) (layer F.Cu) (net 40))
 (segment (start 71.4375 61.43625) (end 72.86625 60.0075) (width 0.25) (layer F.Cu) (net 40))
 (segment (start 71.4375 69.05625) (end 90.4875 69.05625) (width 0.25) (layer F.Cu) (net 5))
 (segment (start 90.4875 69.05625) (end 109.5375 69.05625) (width 0.25) (layer F.Cu) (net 5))
 (segment (start 110.5875 69.05625) (end 127.79375 69.05625) (width 0.25) (layer F.Cu) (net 5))
 (segment (start 109.5375 69.05625) (end 110.5875 69.05625) (width 0.25) (layer F.Cu) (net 5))
 (segment (start 127.79375 72.86625) (end 130.4925 75.565) (width 0.25) (layer B.Cu) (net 5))
 (segment (start 127.79375 69.05625) (end 127.79375 72.86625) (width 0.25) (layer B.Cu) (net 5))
 (segment (start 91.91625 60.0075) (end 102.5525 60.0075) (width 0.25) (layer F.Cu) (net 39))
 (segment (start 90.4875 61.43625) (end 91.91625 60.0075) (width 0.25) (layer F.Cu) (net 39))
 (segment (start 110.96625 60.0075) (end 121.6025 60.0075) (width 0.25) (layer F.Cu) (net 38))
 (segment (start 109.5375 61.43625) (end 110.96625 60.0075) (width 0.25) (layer F.Cu) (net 38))
 (segment (start 129.2225 60.0075) (end 140.6525 60.0075) (width 0.25) (layer F.Cu) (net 37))
 (segment (start 127.79375 61.43625) (end 129.2225 60.0075) (width 0.25) (layer F.Cu) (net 37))
 (segment (start 72.86625 79.0575) (end 83.5025 79.0575) (width 0.25) (layer F.Cu) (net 36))
 (segment (start 71.4375 80.48625) (end 72.86625 79.0575) (width 0.25) (layer F.Cu) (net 36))
 (segment (start 71.4375 88.10625) (end 90.4875 88.10625) (width 0.25) (layer F.Cu) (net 10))
 (segment (start 90.4875 88.10625) (end 109.5375 88.10625) (width 0.25) (layer F.Cu) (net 10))
 (segment (start 109.5375 88.10625) (end 127.79375 88.10625) (width 0.25) (layer F.Cu) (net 10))
 (segment (start 130.33375 88.10625) (end 130.4925 88.265) (width 0.25) (layer F.Cu) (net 10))
 (segment (start 127.79375 88.10625) (end 130.33375 88.10625) (width 0.25) (layer F.Cu) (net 10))
 (segment (start 91.91625 79.0575) (end 102.5525 79.0575) (width 0.25) (layer F.Cu) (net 35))
 (segment (start 90.4875 80.48625) (end 91.91625 79.0575) (width 0.25) (layer F.Cu) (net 35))
 (segment (start 110.96625 79.0575) (end 121.6025 79.0575) (width 0.25) (layer F.Cu) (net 34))
 (segment (start 109.5375 80.48625) (end 110.96625 79.0575) (width 0.25) (layer F.Cu) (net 34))
 (segment (start 139.06151 79.0575) (end 140.6525 79.0575) (width 0.25) (layer F.Cu) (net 33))
 (segment (start 128.760001 79.519999) (end 138.599011 79.519999) (width 0.25) (layer F.Cu) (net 33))
 (segment (start 138.599011 79.519999) (end 139.06151 79.0575) (width 0.25) (layer F.Cu) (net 33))
 (segment (start 127.79375 80.48625) (end 128.760001 79.519999) (width 0.25) (layer F.Cu) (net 33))
 (segment (start 72.86625 98.1075) (end 83.5025 98.1075) (width 0.25) (layer F.Cu) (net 32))
 (segment (start 71.4375 99.53625) (end 72.86625 98.1075) (width 0.25) (layer F.Cu) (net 32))
 (segment (start 71.4375 107.15625) (end 90.4875 107.15625) (width 0.25) (layer F.Cu) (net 12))
 (segment (start 90.4875 107.15625) (end 109.5375 107.15625) (width 0.25) (layer F.Cu) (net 12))
 (segment (start 109.5375 107.15625) (end 128.5875 107.15625) (width 0.25) (layer F.Cu) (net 12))
 (segment (start 130.4925 94.47637) (end 130.4925 93.345) (width 0.25) (layer B.Cu) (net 12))
 (segment (start 130.4925 106.30125) (end 130.4925 94.47637) (width 0.25) (layer B.Cu) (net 12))
 (segment (start 129.6375 107.15625) (end 130.4925 106.30125) (width 0.25) (layer B.Cu) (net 12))
 (segment (start 128.5875 107.15625) (end 129.6375 107.15625) (width 0.25) (layer B.Cu) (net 12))
 (segment (start 91.91625 98.1075) (end 102.5525 98.1075) (width 0.25) (layer F.Cu) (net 31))
 (segment (start 90.4875 99.53625) (end 91.91625 98.1075) (width 0.25) (layer F.Cu) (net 31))
 (segment (start 110.96625 98.1075) (end 121.6025 98.1075) (width 0.25) (layer F.Cu) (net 30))
 (segment (start 109.5375 99.53625) (end 110.96625 98.1075) (width 0.25) (layer F.Cu) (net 30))
 (segment (start 130.01625 98.1075) (end 140.6525 98.1075) (width 0.25) (layer F.Cu) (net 29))
 (segment (start 128.5875 99.53625) (end 130.01625 98.1075) (width 0.25) (layer F.Cu) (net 29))
 (segment (start 72.86625 117.1575) (end 83.5025 117.1575) (width 0.25) (layer F.Cu) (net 28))
 (segment (start 71.4375 118.58625) (end 72.86625 117.1575) (width 0.25) (layer F.Cu) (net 28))
 (segment (start 71.4375 126.20625) (end 90.4875 126.20625) (width 0.25) (layer F.Cu) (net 9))
 (segment (start 90.4875 126.20625) (end 109.5375 126.20625) (width 0.25) (layer F.Cu) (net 9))
 (segment (start 109.5375 126.20625) (end 128.5875 126.20625) (width 0.25) (layer F.Cu) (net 9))
 (segment (start 131.292499 86.524999) (end 130.4925 85.725) (width 0.25) (layer B.Cu) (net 9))
 (segment (start 131.617501 86.850001) (end 131.292499 86.524999) (width 0.25) (layer B.Cu) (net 9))
 (segment (start 131.617501 122.126249) (end 131.617501 86.850001) (width 0.25) (layer B.Cu) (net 9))
 (segment (start 128.5875 125.15625) (end 131.617501 122.126249) (width 0.25) (layer B.Cu) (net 9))
 (segment (start 128.5875 126.20625) (end 128.5875 125.15625) (width 0.25) (layer B.Cu) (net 9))
 (segment (start 91.91625 117.1575) (end 102.5525 117.1575) (width 0.25) (layer F.Cu) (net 27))
 (segment (start 90.4875 118.58625) (end 91.91625 117.1575) (width 0.25) (layer F.Cu) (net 27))
 (segment (start 110.96625 117.1575) (end 121.6025 117.1575) (width 0.25) (layer F.Cu) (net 26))
 (segment (start 109.5375 118.58625) (end 110.96625 117.1575) (width 0.25) (layer F.Cu) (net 26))
 (segment (start 130.01625 117.1575) (end 140.6525 117.1575) (width 0.25) (layer F.Cu) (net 25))
 (segment (start 128.5875 118.58625) (end 130.01625 117.1575) (width 0.25) (layer F.Cu) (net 25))
 (segment (start 77.1525 62.5475) (end 77.1525 81.5975) (width 0.25) (layer B.Cu) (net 6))
 (segment (start 77.1525 83.18849) (end 77.1525 100.6475) (width 0.25) (layer B.Cu) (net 6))
 (segment (start 77.1525 81.5975) (end 77.1525 83.18849) (width 0.25) (layer B.Cu) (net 6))
 (segment (start 77.1525 102.23849) (end 77.1525 119.6975) (width 0.25) (layer B.Cu) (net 6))
 (segment (start 77.1525 100.6475) (end 77.1525 102.23849) (width 0.25) (layer B.Cu) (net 6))
 (segment (start 129.692501 77.305001) (end 130.4925 78.105) (width 0.25) (layer F.Cu) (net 6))
 (segment (start 92.003747 77.305001) (end 129.692501 77.305001) (width 0.25) (layer F.Cu) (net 6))
 (segment (start 77.1525 81.5975) (end 87.711248 81.5975) (width 0.25) (layer F.Cu) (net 6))
 (segment (start 87.711248 81.5975) (end 92.003747 77.305001) (width 0.25) (layer F.Cu) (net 6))
 (segment (start 96.2025 64.13849) (end 96.2025 81.5975) (width 0.25) (layer B.Cu) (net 7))
 (segment (start 96.2025 62.5475) (end 96.2025 64.13849) (width 0.25) (layer B.Cu) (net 7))
 (segment (start 96.2025 81.5975) (end 96.2025 100.6475) (width 0.25) (layer B.Cu) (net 7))
 (segment (start 96.2025 102.23849) (end 96.2025 119.6975) (width 0.25) (layer B.Cu) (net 7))
 (segment (start 96.2025 100.6475) (end 96.2025 102.23849) (width 0.25) (layer B.Cu) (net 7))
 (segment (start 129.692501 81.444999) (end 130.4925 80.645) (width 0.25) (layer F.Cu) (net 7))
 (segment (start 114.525399 86.456401) (end 124.681099 86.456401) (width 0.25) (layer F.Cu) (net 7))
 (segment (start 109.680249 81.611251) (end 114.525399 86.456401) (width 0.25) (layer F.Cu) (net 7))
 (segment (start 124.681099 86.456401) (end 129.692501 81.444999) (width 0.25) (layer F.Cu) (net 7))
 (segment (start 97.807241 81.611251) (end 109.680249 81.611251) (width 0.25) (layer F.Cu) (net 7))
 (segment (start 97.79349 81.5975) (end 97.807241 81.611251) (width 0.25) (layer F.Cu) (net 7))
 (segment (start 96.2025 81.5975) (end 97.79349 81.5975) (width 0.25) (layer F.Cu) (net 7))
 (segment (start 115.2525 62.5475) (end 115.2525 81.5975) (width 0.25) (layer B.Cu) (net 11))
 (segment (start 115.2525 83.18849) (end 115.2525 100.6475) (width 0.25) (layer B.Cu) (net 11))
 (segment (start 115.2525 81.5975) (end 115.2525 83.18849) (width 0.25) (layer B.Cu) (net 11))
 (segment (start 115.2525 102.23849) (end 115.2525 119.6975) (width 0.25) (layer B.Cu) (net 11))
 (segment (start 115.2525 100.6475) (end 115.2525 102.23849) (width 0.25) (layer B.Cu) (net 11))
 (segment (start 125.095 90.805) (end 130.4925 90.805) (width 0.25) (layer B.Cu) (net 11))
 (segment (start 115.2525 100.6475) (end 125.095 90.805) (width 0.25) (layer B.Cu) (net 11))
 (segment (start 134.3025 64.13849) (end 134.3025 81.5975) (width 0.25) (layer B.Cu) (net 13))
 (segment (start 134.3025 62.5475) (end 134.3025 64.13849) (width 0.25) (layer B.Cu) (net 13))
 (segment (start 134.3025 83.18849) (end 134.3025 100.6475) (width 0.25) (layer B.Cu) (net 13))
 (segment (start 134.3025 81.5975) (end 134.3025 83.18849) (width 0.25) (layer B.Cu) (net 13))
 (segment (start 134.3025 102.23849) (end 134.3025 119.6975) (width 0.25) (layer B.Cu) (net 13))
 (segment (start 134.3025 100.6475) (end 134.3025 102.23849) (width 0.25) (layer B.Cu) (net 13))
 (segment (start 145.7325 94.47637) (end 145.7325 93.345) (width 0.25) (layer F.Cu) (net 13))
 (segment (start 145.7325 95.173502) (end 145.7325 94.47637) (width 0.25) (layer F.Cu) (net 13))
 (segment (start 140.258502 100.6475) (end 145.7325 95.173502) (width 0.25) (layer F.Cu) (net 13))
 (segment (start 134.3025 100.6475) (end 140.258502 100.6475) (width 0.25) (layer F.Cu) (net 13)))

